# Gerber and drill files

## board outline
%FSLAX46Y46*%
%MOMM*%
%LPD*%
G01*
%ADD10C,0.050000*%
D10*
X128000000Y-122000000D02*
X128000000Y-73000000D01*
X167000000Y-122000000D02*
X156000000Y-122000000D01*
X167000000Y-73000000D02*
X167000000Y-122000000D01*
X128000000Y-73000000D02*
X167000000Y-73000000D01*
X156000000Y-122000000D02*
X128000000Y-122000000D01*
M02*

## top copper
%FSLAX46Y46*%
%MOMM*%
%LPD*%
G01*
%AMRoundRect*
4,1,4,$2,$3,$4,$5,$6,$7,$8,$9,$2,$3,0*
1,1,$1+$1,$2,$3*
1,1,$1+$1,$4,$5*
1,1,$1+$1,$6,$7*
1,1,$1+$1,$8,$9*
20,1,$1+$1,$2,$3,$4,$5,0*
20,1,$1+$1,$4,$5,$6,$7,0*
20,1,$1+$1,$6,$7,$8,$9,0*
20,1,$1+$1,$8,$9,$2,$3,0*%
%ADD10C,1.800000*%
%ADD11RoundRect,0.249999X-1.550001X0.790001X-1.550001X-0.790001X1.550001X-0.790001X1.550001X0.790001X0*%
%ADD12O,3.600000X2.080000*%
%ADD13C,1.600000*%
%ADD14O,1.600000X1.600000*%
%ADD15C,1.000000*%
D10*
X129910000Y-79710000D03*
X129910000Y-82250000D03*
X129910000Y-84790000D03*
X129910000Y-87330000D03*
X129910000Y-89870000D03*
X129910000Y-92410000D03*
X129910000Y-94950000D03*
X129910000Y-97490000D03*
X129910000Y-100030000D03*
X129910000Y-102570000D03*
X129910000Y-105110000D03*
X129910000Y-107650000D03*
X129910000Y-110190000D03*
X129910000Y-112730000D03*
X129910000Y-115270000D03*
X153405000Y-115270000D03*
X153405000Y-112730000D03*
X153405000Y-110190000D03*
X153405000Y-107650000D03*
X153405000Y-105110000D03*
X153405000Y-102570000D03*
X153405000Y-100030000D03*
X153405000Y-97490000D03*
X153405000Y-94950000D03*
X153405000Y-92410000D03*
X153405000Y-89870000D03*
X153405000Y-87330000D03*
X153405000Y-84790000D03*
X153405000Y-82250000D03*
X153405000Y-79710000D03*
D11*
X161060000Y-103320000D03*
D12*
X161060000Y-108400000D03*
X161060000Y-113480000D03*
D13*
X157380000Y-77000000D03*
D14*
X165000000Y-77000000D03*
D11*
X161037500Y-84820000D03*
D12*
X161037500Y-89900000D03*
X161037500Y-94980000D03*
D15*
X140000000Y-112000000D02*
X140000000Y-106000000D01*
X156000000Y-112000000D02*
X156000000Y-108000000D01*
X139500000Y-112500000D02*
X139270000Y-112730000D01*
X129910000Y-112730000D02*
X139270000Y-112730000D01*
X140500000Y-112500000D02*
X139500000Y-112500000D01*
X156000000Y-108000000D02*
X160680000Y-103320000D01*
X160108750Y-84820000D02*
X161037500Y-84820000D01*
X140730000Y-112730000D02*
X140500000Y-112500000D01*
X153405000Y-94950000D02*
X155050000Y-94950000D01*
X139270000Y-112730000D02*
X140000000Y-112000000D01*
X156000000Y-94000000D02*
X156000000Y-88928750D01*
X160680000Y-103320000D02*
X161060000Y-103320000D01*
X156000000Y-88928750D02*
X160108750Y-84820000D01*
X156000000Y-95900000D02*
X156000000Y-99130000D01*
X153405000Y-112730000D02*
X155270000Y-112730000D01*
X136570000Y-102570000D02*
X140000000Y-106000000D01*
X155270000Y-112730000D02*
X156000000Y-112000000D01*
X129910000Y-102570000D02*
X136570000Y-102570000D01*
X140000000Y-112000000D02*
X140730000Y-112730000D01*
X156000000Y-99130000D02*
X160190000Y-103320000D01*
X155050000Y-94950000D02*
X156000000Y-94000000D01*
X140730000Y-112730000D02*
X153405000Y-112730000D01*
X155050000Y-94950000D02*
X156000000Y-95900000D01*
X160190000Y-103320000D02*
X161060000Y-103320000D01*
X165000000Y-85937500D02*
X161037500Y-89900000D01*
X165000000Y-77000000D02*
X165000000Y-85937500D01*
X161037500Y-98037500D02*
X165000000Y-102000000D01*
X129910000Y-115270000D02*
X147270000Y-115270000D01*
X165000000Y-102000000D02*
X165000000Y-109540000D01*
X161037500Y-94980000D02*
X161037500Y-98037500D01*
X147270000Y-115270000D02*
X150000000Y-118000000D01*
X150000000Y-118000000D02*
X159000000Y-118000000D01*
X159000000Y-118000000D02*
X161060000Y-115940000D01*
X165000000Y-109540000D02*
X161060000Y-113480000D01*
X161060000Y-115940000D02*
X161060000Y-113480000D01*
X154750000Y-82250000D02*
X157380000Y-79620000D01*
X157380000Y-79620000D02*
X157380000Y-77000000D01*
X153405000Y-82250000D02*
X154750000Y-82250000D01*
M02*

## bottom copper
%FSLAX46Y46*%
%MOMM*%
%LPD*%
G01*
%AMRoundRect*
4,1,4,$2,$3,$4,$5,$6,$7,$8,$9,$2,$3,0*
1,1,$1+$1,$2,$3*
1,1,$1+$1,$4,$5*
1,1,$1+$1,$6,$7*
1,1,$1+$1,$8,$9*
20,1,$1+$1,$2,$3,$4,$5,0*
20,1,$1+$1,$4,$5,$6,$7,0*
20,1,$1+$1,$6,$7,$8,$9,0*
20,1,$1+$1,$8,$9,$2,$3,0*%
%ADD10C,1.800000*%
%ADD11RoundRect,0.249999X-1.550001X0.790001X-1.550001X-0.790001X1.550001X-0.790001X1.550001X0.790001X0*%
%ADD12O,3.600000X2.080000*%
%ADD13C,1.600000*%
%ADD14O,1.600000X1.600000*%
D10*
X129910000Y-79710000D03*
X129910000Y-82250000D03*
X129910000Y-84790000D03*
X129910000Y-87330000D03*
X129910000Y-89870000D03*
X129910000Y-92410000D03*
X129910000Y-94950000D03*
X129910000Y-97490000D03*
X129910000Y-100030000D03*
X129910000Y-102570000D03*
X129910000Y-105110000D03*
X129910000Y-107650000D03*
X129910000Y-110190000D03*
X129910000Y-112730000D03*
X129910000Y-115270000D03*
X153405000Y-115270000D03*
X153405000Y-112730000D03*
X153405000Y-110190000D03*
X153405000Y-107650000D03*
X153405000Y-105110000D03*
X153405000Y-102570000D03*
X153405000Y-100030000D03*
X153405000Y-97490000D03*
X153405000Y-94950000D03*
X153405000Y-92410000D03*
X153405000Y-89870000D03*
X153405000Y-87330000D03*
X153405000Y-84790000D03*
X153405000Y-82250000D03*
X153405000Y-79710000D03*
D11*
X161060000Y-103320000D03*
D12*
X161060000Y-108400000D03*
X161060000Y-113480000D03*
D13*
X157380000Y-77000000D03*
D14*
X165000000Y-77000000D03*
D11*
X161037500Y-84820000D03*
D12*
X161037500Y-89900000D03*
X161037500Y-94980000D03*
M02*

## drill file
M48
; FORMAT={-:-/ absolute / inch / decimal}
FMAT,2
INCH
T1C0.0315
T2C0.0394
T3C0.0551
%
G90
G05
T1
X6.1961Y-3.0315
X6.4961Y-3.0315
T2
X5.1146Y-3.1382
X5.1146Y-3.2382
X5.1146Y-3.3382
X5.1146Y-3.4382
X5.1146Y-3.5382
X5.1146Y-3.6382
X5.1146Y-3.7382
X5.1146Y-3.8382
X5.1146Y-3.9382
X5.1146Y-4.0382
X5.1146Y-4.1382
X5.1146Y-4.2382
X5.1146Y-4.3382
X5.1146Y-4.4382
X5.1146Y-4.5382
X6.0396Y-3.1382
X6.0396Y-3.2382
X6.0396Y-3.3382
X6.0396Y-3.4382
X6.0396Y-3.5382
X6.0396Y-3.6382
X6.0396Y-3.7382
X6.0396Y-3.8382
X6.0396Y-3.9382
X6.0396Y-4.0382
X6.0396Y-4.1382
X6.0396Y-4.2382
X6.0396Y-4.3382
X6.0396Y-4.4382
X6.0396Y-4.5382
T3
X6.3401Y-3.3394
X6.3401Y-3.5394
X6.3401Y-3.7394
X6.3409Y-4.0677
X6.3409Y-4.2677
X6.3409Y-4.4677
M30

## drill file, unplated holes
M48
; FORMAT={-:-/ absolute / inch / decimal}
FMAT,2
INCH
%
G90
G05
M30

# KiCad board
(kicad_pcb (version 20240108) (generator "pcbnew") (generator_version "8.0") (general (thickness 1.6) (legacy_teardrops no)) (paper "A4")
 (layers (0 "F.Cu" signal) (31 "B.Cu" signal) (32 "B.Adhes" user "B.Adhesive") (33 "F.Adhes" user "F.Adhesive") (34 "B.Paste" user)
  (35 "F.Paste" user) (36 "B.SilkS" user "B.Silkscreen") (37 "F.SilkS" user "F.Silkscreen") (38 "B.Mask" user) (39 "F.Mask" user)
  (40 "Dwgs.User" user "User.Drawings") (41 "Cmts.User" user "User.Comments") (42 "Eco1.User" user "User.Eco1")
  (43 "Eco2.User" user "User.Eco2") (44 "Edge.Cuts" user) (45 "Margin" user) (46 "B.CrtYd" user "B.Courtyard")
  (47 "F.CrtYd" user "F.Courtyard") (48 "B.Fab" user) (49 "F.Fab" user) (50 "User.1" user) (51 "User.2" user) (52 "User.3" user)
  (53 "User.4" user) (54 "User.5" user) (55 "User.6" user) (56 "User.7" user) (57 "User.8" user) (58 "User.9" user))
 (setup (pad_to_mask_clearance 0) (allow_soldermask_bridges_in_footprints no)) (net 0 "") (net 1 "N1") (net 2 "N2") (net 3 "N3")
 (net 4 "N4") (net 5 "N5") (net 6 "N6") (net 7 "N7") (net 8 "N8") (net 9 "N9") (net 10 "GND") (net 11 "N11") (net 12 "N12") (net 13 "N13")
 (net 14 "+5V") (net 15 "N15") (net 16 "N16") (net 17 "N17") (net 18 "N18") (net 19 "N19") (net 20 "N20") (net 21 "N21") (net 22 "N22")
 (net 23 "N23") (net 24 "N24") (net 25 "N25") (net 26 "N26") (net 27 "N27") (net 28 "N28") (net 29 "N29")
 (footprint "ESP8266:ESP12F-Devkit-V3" (layer "F.Cu") (at 141.975 98.76)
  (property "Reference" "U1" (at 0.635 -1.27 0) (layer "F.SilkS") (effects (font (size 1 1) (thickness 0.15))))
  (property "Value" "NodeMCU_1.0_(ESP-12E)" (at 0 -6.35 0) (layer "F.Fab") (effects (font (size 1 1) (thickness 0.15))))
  (pad "1" thru_hole circle (at -12.065 -19.05) (size 1.8 1.8) (drill 1) (layers "*.Cu" "*.Mask") (remove_unused_layers no) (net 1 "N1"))
  (pad "2" thru_hole circle (at -12.065 -16.51) (size 1.8 1.8) (drill 1) (layers "*.Cu" "*.Mask") (remove_unused_layers no) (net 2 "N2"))
  (pad "3" thru_hole circle (at -12.065 -13.97) (size 1.8 1.8) (drill 1) (layers "*.Cu" "*.Mask") (remove_unused_layers no) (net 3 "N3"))
  (pad "4" thru_hole circle (at -12.065 -11.43) (size 1.8 1.8) (drill 1) (layers "*.Cu" "*.Mask") (remove_unused_layers no) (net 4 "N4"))
  (pad "5" thru_hole circle (at -12.065 -8.89) (size 1.8 1.8) (drill 1) (layers "*.Cu" "*.Mask") (remove_unused_layers no) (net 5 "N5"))
  (pad "6" thru_hole circle (at -12.065 -6.35) (size 1.8 1.8) (drill 1) (layers "*.Cu" "*.Mask") (remove_unused_layers no) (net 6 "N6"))
  (pad "7" thru_hole circle (at -12.065 -3.81) (size 1.8 1.8) (drill 1) (layers "*.Cu" "*.Mask") (remove_unused_layers no) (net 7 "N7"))
  (pad "8" thru_hole circle (at -12.065 -1.27) (size 1.8 1.8) (drill 1) (layers "*.Cu" "*.Mask") (remove_unused_layers no) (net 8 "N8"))
  (pad "9" thru_hole circle (at -12.065 1.27) (size 1.8 1.8) (drill 1) (layers "*.Cu" "*.Mask") (remove_unused_layers no) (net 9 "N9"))
  (pad "10" thru_hole circle (at -12.065 3.81) (size 1.8 1.8) (drill 1) (layers "*.Cu" "*.Mask") (remove_unused_layers no) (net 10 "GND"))
  (pad "11" thru_hole circle (at -12.065 6.35) (size 1.8 1.8) (drill 1) (layers "*.Cu" "*.Mask") (remove_unused_layers no) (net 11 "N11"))
  (pad "12" thru_hole circle (at -12.065 8.89) (size 1.8 1.8) (drill 1) (layers "*.Cu" "*.Mask") (remove_unused_layers no) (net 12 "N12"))
  (pad "13" thru_hole circle (at -12.065 11.43) (size 1.8 1.8) (drill 1) (layers "*.Cu" "*.Mask") (remove_unused_layers no) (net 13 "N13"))
  (pad "14" thru_hole circle (at -12.065 13.97) (size 1.8 1.8) (drill 1) (layers "*.Cu" "*.Mask") (remove_unused_layers no) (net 10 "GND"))
  (pad "15" thru_hole circle (at -12.065 16.51) (size 1.8 1.8) (drill 1) (layers "*.Cu" "*.Mask") (remove_unused_layers no) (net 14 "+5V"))
  (pad "16" thru_hole circle (at 11.43 16.51) (size 1.8 1.8) (drill 1) (layers "*.Cu" "*.Mask") (remove_unused_layers no) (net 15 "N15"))
  (pad "17" thru_hole circle (at 11.43 13.97) (size 1.8 1.8) (drill 1) (layers "*.Cu" "*.Mask") (remove_unused_layers no) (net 10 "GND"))
  (pad "18" thru_hole circle (at 11.43 11.43) (size 1.8 1.8) (drill 1) (layers "*.Cu" "*.Mask") (remove_unused_layers no) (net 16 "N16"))
  (pad "19" thru_hole circle (at 11.43 8.89) (size 1.8 1.8) (drill 1) (layers "*.Cu" "*.Mask") (remove_unused_layers no) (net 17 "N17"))
  (pad "20" thru_hole circle (at 11.43 6.35) (size 1.8 1.8) (drill 1) (layers "*.Cu" "*.Mask") (remove_unused_layers no) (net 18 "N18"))
  (pad "21" thru_hole circle (at 11.43 3.81) (size 1.8 1.8) (drill 1) (layers "*.Cu" "*.Mask") (remove_unused_layers no) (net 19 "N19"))
  (pad "22" thru_hole circle (at 11.43 1.27) (size 1.8 1.8) (drill 1) (layers "*.Cu" "*.Mask") (remove_unused_layers no) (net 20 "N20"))
  (pad "23" thru_hole circle (at 11.43 -1.27) (size 1.8 1.8) (drill 1) (layers "*.Cu" "*.Mask") (remove_unused_layers no) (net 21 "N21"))
  (pad "24" thru_hole circle (at 11.43 -3.81) (size 1.8 1.8) (drill 1) (layers "*.Cu" "*.Mask") (remove_unused_layers no) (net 10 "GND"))
  (pad "25" thru_hole circle (at 11.43 -6.35) (size 1.8 1.8) (drill 1) (layers "*.Cu" "*.Mask") (remove_unused_layers no) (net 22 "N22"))
  (pad "26" thru_hole circle (at 11.43 -8.89) (size 1.8 1.8) (drill 1) (layers "*.Cu" "*.Mask") (remove_unused_layers no) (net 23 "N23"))
  (pad "27" thru_hole circle (at 11.43 -11.43) (size 1.8 1.8) (drill 1) (layers "*.Cu" "*.Mask") (remove_unused_layers no) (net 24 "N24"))
  (pad "28" thru_hole circle (at 11.43 -13.97) (size 1.8 1.8) (drill 1) (layers "*.Cu" "*.Mask") (remove_unused_layers no) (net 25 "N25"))
  (pad "29" thru_hole circle (at 11.43 -16.51) (size 1.8 1.8) (drill 1) (layers "*.Cu" "*.Mask") (remove_unused_layers no) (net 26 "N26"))
  (pad "30" thru_hole circle (at 11.43 -19.05) (size 1.8 1.8) (drill 1) (layers "*.Cu" "*.Mask") (remove_unused_layers no) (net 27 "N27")))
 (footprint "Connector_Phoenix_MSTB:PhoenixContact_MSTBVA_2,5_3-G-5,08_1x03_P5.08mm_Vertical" (layer "F.Cu") (at 161.06 103.32 -90)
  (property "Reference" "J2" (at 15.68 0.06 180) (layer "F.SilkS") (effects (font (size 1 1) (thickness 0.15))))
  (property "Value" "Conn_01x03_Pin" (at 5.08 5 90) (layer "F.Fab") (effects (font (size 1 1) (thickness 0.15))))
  (pad "1" thru_hole roundrect (at 0 0 270) (size 2.08 3.6) (drill 1.4) (layers "*.Cu" "*.Mask") (remove_unused_layers no)
   (roundrect_rratio 0.120192) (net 10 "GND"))
  (pad "2" thru_hole oval (at 5.08 0 270) (size 2.08 3.6) (drill 1.4) (layers "*.Cu" "*.Mask") (remove_unused_layers no) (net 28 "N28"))
  (pad "3" thru_hole oval (at 10.16 0 270) (size 2.08 3.6) (drill 1.4) (layers "*.Cu" "*.Mask") (remove_unused_layers no) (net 14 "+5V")))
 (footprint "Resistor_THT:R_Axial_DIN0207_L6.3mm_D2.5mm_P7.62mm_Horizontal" (layer "F.Cu") (at 157.38 77)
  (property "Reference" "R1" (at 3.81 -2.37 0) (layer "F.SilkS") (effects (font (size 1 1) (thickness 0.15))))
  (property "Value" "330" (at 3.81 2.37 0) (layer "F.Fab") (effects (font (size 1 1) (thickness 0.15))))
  (pad "1" thru_hole circle (at 0 0) (size 1.6 1.6) (drill 0.8) (layers "*.Cu" "*.Mask") (remove_unused_layers no) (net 26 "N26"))
  (pad "2" thru_hole oval (at 7.62 0) (size 1.6 1.6) (drill 0.8) (layers "*.Cu" "*.Mask") (remove_unused_layers no) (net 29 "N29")))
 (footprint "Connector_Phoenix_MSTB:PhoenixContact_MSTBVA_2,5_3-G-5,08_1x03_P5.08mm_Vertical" (layer "F.Cu") (at 161.0375 84.82 -90)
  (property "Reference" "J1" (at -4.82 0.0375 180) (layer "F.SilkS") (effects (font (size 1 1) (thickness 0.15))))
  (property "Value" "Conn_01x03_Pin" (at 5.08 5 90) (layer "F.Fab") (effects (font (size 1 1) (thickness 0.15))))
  (pad "1" thru_hole roundrect (at 0 0 270) (size 2.08 3.6) (drill 1.4) (layers "*.Cu" "*.Mask") (remove_unused_layers no)
   (roundrect_rratio 0.120192) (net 10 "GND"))
  (pad "2" thru_hole oval (at 5.08 0 270) (size 2.08 3.6) (drill 1.4) (layers "*.Cu" "*.Mask") (remove_unused_layers no) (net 29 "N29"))
  (pad "3" thru_hole oval (at 10.16 0 270) (size 2.08 3.6) (drill 1.4) (layers "*.Cu" "*.Mask") (remove_unused_layers no) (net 14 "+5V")))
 (gr_line (start 128 122) (end 128 73) (stroke (width 0.05) (type default)) (layer "Edge.Cuts"))
 (gr_line (start 167 122) (end 156 122) (stroke (width 0.05) (type default)) (layer "Edge.Cuts"))
 (gr_line (start 167 73) (end 167 122) (stroke (width 0.05) (type default)) (layer "Edge.Cuts"))
 (gr_line (start 128 73) (end 167 73) (stroke (width 0.05) (type default)) (layer "Edge.Cuts"))
 (gr_line (start 156 122) (end 128 122) (stroke (width 0.05) (type default)) (layer "Edge.Cuts"))
 (segment (start 140 112) (end 140 106) (width 1) (layer "F.Cu") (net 10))
 (segment (start 156 112) (end 156 108) (width 1) (layer "F.Cu") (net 10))
 (segment (start 139.5 112.5) (end 139.27 112.73) (width 1) (layer "F.Cu") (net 10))
 (segment (start 129.91 112.73) (end 139.27 112.73) (width 1) (layer "F.Cu") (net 10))
 (segment (start 140.5 112.5) (end 139.5 112.5) (width 1) (layer "F.Cu") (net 10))
 (segment (start 156 108) (end 160.68 103.32) (width 1) (layer "F.Cu") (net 10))
 (segment (start 160.10875 84.82) (end 161.0375 84.82) (width 1) (layer "F.Cu") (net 10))
 (segment (start 140.73 112.73) (end 140.5 112.5) (width 1) (layer "F.Cu") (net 10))
 (segment (start 153.405 94.95) (end 155.05 94.95) (width 1) (layer "F.Cu") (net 10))
 (segment (start 139.27 112.73) (end 140 112) (width 1) (layer "F.Cu") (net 10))
 (segment (start 156 94) (end 156 88.92875) (width 1) (layer "F.Cu") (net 10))
 (segment (start 160.68 103.32) (end 161.06 103.32) (width 1) (layer "F.Cu") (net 10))
 (segment (start 156 88.92875) (end 160.10875 84.82) (width 1) (layer "F.Cu") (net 10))
 (segment (start 156 95.9) (end 156 99.13) (width 1) (layer "F.Cu") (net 10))
 (segment (start 153.405 112.73) (end 155.27 112.73) (width 1) (layer "F.Cu") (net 10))
 (segment (start 136.57 102.57) (end 140 106) (width 1) (layer "F.Cu") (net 10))
 (segment (start 155.27 112.73) (end 156 112) (width 1) (layer "F.Cu") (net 10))
 (segment (start 129.91 102.57) (end 136.57 102.57) (width 1) (layer "F.Cu") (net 10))
 (segment (start 140 112) (end 140.73 112.73) (width 1) (layer "F.Cu") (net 10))
 (segment (start 156 99.13) (end 160.19 103.32) (width 1) (layer "F.Cu") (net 10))
 (segment (start 155.05 94.95) (end 156 94) (width 1) (layer "F.Cu") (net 10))
 (segment (start 140.73 112.73) (end 153.405 112.73) (width 1) (layer "F.Cu") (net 10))
 (segment (start 155.05 94.95) (end 156 95.9) (width 1) (layer "F.Cu") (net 10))
 (segment (start 160.19 103.32) (end 161.06 103.32) (width 1) (layer "F.Cu") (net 10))
 (segment (start 165 85.9375) (end 161.0375 89.9) (width 1) (layer "F.Cu") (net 29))
 (segment (start 165 77) (end 165 85.9375) (width 1) (layer "F.Cu") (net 29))
 (segment (start 161.0375 98.0375) (end 165 102) (width 1) (layer "F.Cu") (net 14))
 (segment (start 129.91 115.27) (end 147.27 115.27) (width 1) (layer "F.Cu") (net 14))
 (segment (start 165 102) (end 165 109.54) (width 1) (layer "F.Cu") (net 14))
 (segment (start 161.0375 94.98) (end 161.0375 98.0375) (width 1) (layer "F.Cu") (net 14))
 (segment (start 147.27 115.27) (end 150 118) (width 1) (layer "F.Cu") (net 14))
 (segment (start 150 118) (end 159 118) (width 1) (layer "F.Cu") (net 14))
 (segment (start 159 118) (end 161.06 115.94) (width 1) (layer "F.Cu") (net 14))
 (segment (start 165 109.54) (end 161.06 113.48) (width 1) (layer "F.Cu") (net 14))
 (segment (start 161.06 115.94) (end 161.06 113.48) (width 1) (layer "F.Cu") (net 14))
 (segment (start 154.75 82.25) (end 157.38 79.62) (width 1) (layer "F.Cu") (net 26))
 (segment (start 157.38 79.62) (end 157.38 77) (width 1) (layer "F.Cu") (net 26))
 (segment (start 153.405 82.25) (end 154.75 82.25) (width 1) (layer "F.Cu") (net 26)))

